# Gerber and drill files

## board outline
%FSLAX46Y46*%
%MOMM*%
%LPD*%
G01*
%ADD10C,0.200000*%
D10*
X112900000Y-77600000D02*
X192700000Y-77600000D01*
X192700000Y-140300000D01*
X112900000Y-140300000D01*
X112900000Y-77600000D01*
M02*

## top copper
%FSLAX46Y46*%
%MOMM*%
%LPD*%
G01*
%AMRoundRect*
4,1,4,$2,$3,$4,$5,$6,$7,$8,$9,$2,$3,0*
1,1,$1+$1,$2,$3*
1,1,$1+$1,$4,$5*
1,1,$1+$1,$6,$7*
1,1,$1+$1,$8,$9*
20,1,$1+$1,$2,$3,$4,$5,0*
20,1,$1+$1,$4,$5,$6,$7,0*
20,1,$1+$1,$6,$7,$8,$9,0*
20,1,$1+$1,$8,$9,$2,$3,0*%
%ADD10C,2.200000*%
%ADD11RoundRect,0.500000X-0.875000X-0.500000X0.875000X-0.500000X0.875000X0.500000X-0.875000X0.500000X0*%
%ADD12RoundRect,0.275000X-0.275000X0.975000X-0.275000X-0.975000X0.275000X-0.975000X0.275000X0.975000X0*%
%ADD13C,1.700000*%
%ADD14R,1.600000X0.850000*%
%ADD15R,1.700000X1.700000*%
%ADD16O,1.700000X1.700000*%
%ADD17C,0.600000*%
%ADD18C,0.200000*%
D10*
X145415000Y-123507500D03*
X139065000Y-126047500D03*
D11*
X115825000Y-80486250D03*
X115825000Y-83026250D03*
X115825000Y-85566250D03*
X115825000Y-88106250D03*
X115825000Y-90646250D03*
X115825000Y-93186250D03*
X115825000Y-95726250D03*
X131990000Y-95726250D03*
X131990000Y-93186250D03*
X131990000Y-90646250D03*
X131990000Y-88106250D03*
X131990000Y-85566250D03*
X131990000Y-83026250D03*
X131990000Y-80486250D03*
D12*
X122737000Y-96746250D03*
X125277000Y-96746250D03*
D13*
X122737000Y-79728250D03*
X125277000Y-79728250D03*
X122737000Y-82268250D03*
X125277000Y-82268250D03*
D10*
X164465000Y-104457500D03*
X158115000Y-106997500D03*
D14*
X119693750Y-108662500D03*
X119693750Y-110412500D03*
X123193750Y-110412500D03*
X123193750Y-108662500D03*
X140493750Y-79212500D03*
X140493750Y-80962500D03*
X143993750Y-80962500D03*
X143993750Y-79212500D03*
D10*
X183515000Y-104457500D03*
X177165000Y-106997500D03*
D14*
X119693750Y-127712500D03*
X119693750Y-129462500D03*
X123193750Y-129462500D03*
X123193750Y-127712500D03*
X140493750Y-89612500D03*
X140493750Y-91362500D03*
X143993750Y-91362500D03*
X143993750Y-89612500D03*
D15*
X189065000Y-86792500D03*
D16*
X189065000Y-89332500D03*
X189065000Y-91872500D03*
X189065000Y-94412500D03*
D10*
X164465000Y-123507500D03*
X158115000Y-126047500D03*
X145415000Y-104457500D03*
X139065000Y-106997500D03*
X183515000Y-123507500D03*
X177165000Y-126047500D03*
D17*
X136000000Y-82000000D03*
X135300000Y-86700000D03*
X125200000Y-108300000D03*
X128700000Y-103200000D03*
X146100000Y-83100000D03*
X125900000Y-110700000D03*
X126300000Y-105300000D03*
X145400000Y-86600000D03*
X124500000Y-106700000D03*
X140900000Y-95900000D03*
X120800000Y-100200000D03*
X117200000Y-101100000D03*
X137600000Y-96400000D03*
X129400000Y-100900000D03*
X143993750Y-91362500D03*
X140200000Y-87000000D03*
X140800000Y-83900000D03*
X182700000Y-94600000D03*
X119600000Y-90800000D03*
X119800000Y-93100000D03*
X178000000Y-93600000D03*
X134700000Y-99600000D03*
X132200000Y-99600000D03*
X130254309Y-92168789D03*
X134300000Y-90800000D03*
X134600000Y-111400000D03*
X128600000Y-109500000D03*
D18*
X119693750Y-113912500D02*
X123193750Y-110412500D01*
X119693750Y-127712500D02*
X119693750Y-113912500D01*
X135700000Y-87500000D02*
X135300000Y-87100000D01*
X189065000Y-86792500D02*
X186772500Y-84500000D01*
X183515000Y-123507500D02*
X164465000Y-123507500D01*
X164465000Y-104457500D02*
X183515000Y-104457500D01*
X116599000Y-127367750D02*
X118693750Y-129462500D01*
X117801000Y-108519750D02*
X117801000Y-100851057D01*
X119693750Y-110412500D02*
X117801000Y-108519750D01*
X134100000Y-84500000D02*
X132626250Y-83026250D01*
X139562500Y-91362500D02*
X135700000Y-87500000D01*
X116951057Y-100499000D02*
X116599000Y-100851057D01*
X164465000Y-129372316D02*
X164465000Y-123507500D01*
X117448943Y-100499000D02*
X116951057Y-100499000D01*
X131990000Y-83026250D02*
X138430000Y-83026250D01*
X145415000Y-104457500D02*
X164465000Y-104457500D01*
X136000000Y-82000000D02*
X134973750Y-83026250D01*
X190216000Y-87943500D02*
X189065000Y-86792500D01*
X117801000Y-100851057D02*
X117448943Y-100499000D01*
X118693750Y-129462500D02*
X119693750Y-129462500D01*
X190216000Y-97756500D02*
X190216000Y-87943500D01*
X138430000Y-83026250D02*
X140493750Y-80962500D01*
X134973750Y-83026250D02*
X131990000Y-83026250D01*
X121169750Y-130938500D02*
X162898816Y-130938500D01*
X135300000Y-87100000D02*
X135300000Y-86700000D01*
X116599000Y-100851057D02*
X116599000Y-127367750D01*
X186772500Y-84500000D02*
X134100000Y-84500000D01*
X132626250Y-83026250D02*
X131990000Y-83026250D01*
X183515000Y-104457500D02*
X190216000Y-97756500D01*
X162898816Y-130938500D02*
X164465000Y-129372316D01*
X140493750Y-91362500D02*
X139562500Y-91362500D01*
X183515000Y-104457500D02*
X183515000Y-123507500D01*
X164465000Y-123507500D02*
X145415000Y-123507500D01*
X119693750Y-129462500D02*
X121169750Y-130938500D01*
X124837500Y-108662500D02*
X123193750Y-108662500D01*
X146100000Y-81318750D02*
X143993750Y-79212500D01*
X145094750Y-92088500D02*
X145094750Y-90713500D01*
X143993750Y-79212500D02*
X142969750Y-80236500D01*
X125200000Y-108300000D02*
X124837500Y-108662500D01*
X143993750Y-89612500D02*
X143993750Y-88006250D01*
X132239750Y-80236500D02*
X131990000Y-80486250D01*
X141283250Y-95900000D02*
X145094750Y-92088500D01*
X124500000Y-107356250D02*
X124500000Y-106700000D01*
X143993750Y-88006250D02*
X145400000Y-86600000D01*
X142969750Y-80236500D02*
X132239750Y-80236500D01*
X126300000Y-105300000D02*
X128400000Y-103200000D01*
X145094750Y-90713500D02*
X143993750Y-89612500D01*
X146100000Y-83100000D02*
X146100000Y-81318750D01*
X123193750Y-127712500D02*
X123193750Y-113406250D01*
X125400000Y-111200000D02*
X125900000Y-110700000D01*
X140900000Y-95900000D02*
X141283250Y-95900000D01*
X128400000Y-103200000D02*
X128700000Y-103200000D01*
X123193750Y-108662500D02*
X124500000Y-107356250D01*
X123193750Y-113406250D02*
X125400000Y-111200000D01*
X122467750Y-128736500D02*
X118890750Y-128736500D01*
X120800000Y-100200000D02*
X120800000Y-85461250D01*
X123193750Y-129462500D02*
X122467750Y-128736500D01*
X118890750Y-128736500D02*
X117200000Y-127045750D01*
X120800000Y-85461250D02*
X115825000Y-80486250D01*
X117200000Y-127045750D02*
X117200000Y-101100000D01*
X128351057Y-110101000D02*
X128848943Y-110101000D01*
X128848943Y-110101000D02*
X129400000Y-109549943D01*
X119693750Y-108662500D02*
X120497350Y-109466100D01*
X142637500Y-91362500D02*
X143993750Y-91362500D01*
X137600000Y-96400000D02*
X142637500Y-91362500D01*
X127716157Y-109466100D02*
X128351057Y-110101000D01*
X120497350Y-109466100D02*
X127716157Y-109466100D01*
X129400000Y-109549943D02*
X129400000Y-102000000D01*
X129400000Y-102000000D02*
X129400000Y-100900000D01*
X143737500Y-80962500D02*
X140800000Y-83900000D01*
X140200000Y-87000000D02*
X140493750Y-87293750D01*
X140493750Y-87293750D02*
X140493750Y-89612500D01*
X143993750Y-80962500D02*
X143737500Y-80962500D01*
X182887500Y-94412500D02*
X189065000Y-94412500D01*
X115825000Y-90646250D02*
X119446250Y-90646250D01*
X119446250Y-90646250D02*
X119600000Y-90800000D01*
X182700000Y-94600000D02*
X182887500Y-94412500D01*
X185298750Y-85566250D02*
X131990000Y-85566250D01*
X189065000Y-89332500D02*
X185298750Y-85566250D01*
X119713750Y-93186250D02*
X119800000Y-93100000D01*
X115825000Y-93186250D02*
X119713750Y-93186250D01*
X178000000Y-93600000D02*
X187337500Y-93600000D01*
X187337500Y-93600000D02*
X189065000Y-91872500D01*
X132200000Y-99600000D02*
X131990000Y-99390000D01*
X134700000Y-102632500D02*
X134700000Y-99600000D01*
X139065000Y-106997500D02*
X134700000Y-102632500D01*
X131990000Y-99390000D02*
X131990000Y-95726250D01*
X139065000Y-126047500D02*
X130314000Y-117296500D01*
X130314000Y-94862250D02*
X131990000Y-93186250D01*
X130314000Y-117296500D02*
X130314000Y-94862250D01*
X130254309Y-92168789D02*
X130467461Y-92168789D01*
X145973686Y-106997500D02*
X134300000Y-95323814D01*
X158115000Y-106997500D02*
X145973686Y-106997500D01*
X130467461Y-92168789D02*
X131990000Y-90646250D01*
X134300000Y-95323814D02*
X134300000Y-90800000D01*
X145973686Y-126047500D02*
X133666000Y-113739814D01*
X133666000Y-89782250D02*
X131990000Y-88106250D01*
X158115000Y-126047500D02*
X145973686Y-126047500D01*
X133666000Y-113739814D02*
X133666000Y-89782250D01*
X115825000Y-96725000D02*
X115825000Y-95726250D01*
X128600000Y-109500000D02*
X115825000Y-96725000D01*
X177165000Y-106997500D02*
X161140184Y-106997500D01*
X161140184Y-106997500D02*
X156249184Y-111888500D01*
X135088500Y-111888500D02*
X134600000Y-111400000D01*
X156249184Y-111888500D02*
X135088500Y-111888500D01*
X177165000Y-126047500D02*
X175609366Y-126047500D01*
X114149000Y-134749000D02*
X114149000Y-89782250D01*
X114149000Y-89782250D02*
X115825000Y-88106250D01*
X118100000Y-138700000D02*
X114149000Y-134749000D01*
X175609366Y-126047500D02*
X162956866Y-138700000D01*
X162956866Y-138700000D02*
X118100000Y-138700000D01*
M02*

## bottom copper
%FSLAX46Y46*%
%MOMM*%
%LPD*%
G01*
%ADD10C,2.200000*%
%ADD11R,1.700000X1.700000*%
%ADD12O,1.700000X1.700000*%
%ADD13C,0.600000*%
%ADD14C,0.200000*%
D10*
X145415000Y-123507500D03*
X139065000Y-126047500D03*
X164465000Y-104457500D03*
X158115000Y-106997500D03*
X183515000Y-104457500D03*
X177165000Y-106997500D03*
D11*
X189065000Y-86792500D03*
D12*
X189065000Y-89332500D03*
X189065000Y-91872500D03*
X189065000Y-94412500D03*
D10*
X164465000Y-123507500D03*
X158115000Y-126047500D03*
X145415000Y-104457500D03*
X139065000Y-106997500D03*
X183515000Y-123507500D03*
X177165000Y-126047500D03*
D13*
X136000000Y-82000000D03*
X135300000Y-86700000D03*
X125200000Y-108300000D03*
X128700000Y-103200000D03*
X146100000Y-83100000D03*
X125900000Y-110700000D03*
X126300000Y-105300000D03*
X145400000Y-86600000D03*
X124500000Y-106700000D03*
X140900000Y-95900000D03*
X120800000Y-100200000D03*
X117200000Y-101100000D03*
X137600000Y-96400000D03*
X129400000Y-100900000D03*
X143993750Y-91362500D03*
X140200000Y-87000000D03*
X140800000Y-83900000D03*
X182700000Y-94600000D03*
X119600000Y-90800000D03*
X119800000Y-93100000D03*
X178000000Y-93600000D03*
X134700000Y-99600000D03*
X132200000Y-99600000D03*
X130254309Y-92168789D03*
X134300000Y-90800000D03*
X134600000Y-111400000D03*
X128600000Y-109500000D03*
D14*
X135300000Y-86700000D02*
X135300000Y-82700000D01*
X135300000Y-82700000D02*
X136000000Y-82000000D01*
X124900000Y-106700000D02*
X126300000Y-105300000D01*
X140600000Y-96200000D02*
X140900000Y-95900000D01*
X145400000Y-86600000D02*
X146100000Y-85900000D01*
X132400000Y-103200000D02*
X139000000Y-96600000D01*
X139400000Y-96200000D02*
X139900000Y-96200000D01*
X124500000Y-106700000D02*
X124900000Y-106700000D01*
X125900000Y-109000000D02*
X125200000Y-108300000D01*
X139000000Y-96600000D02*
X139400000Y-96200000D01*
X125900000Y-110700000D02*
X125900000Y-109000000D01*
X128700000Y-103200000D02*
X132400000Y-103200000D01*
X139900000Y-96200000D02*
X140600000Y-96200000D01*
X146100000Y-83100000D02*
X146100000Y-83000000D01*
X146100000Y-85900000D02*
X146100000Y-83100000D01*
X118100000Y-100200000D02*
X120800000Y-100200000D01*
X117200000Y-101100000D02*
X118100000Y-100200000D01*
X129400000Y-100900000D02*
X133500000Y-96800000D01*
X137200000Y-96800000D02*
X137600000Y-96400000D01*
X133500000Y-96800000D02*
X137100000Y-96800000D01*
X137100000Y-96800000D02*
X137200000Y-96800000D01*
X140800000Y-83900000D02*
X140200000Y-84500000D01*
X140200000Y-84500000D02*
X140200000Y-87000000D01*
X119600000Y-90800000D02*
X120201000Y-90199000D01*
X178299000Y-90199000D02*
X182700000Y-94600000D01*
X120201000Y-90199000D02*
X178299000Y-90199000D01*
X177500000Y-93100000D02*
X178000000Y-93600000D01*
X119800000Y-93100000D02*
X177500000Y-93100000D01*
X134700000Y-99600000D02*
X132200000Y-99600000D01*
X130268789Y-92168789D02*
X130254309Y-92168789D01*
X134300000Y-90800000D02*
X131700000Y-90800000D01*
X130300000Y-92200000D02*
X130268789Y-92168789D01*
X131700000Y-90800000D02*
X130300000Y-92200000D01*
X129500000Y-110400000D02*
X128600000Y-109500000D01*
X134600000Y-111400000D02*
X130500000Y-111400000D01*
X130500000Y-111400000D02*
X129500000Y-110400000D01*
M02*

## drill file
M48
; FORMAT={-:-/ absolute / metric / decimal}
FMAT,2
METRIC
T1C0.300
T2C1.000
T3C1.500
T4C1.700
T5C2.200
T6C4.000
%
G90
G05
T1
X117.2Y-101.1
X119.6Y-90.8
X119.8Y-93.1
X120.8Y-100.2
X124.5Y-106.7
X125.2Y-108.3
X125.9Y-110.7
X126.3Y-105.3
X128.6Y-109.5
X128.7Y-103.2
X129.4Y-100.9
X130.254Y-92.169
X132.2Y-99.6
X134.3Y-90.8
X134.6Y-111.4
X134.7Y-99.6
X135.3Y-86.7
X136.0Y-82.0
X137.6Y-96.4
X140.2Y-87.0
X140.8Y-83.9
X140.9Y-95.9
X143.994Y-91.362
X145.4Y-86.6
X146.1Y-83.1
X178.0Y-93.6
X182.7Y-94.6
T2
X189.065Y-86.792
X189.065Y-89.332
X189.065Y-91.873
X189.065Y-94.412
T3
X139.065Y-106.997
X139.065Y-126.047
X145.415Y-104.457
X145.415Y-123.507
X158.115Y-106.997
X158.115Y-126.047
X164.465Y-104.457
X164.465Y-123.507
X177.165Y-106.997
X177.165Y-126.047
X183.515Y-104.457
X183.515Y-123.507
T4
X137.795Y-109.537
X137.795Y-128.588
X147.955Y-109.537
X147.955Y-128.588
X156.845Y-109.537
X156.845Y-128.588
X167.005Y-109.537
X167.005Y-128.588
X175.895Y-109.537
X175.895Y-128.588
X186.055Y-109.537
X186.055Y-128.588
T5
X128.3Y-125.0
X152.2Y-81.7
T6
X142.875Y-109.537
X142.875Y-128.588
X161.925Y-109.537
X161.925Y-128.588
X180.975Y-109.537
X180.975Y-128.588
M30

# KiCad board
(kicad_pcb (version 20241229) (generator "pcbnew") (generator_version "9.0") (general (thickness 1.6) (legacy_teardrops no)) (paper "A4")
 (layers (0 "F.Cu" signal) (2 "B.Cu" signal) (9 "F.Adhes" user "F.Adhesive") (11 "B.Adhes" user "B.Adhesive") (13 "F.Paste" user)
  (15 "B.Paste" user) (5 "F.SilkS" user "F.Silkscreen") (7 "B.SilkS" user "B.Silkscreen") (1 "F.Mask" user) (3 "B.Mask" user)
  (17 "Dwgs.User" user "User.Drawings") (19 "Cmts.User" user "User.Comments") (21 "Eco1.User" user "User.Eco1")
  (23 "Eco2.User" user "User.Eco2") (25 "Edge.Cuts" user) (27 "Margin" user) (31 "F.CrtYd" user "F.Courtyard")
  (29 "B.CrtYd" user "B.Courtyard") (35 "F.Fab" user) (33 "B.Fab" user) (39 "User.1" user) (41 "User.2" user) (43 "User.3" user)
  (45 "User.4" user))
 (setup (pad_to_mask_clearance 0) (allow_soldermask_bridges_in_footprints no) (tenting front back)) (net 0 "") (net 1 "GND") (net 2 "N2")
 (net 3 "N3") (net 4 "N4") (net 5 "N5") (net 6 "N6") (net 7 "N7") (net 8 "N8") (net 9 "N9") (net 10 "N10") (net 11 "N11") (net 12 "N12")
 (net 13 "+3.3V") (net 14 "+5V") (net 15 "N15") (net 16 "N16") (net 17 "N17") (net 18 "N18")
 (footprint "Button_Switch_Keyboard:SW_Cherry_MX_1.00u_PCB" (layer "F.Cu") (at 145.415 123.5075)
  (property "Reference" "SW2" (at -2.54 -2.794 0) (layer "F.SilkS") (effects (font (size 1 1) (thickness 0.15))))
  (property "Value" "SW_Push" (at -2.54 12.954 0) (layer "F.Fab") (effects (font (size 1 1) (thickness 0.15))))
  (pad "" np_thru_hole circle (at -7.62 5.08) (size 1.7 1.7) (drill 1.7) (layers "*.Cu" "*.Mask"))
  (pad "" np_thru_hole circle (at -2.54 5.08) (size 4 4) (drill 4) (layers "*.Cu" "*.Mask"))
  (pad "" np_thru_hole circle (at 2.54 5.08) (size 1.7 1.7) (drill 1.7) (layers "*.Cu" "*.Mask"))
  (pad "1" thru_hole circle (at 0 0) (size 2.2 2.2) (drill 1.5) (layers "*.Cu" "*.Mask") (remove_unused_layers no) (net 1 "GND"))
  (pad "2" thru_hole circle (at -6.35 2.54) (size 2.2 2.2) (drill 1.5) (layers "*.Cu" "*.Mask") (remove_unused_layers no) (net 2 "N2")))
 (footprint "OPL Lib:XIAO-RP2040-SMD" (layer "F.Cu") (at 123.825 88.10625)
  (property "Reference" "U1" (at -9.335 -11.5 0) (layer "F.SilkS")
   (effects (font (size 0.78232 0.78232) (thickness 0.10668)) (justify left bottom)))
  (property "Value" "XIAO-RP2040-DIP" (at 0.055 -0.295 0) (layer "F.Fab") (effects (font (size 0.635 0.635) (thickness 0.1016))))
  (pad "1" smd roundrect (at -8 -7.62) (size 2.75 2) (layers "F.Cu" "F.Mask" "F.Paste") (roundrect_rratio 0.25) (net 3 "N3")
   (solder_mask_margin 0.0508) (thermal_bridge_angle 45))
  (pad "2" smd roundrect (at -8 -5.08) (size 2.75 2) (layers "F.Cu" "F.Mask" "F.Paste") (roundrect_rratio 0.25) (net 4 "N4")
   (solder_mask_margin 0.0508) (thermal_bridge_angle 45))
  (pad "3" smd roundrect (at -8 -2.54) (size 2.75 2) (layers "F.Cu" "F.Mask" "F.Paste") (roundrect_rratio 0.25) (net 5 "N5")
   (solder_mask_margin 0.0508) (thermal_bridge_angle 45))
  (pad "4" smd roundrect (at -8 0) (size 2.75 2) (layers "F.Cu" "F.Mask" "F.Paste") (roundrect_rratio 0.25) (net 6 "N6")
   (solder_mask_margin 0.0508) (thermal_bridge_angle 45))
  (pad "5" smd roundrect (at -8 2.54) (size 2.75 2) (layers "F.Cu" "F.Mask" "F.Paste") (roundrect_rratio 0.25) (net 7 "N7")
   (solder_mask_margin 0.0508) (thermal_bridge_angle 45))
  (pad "6" smd roundrect (at -8 5.08) (size 2.75 2) (layers "F.Cu" "F.Mask" "F.Paste") (roundrect_rratio 0.25) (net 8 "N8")
   (solder_mask_margin 0.0508) (thermal_bridge_angle 45))
  (pad "7" smd roundrect (at -8 7.62) (size 2.75 2) (layers "F.Cu" "F.Mask" "F.Paste") (roundrect_rratio 0.25) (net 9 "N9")
   (solder_mask_margin 0.0508) (thermal_bridge_angle 45))
  (pad "8" smd roundrect (at 8.165 7.62) (size 2.75 2) (layers "F.Cu" "F.Mask" "F.Paste") (roundrect_rratio 0.25) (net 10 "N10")
   (solder_mask_margin 0.0508) (thermal_bridge_angle 45))
  (pad "9" smd roundrect (at 8.165 5.08) (size 2.75 2) (layers "F.Cu" "F.Mask" "F.Paste") (roundrect_rratio 0.25) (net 2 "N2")
   (solder_mask_margin 0.0508) (thermal_bridge_angle 45))
  (pad "10" smd roundrect (at 8.165 2.54) (size 2.75 2) (layers "F.Cu" "F.Mask" "F.Paste") (roundrect_rratio 0.25) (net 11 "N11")
   (solder_mask_margin 0.0508) (thermal_bridge_angle 45))
  (pad "11" smd roundrect (at 8.165 0) (size 2.75 2) (layers "F.Cu" "F.Mask" "F.Paste") (roundrect_rratio 0.25) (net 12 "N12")
   (solder_mask_margin 0.0508) (thermal_bridge_angle 45))
  (pad "12" smd roundrect (at 8.165 -2.54) (size 2.75 2) (layers "F.Cu" "F.Mask" "F.Paste") (roundrect_rratio 0.25) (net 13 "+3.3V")
   (solder_mask_margin 0.0508) (thermal_bridge_angle 45))
  (pad "13" smd roundrect (at 8.165 -5.08) (size 2.75 2) (layers "F.Cu" "F.Mask" "F.Paste") (roundrect_rratio 0.25) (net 1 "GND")
   (solder_mask_margin 0.0508) (thermal_bridge_angle 45))
  (pad "14" smd roundrect (at 8.165 -7.62) (size 2.75 2) (layers "F.Cu" "F.Mask" "F.Paste") (roundrect_rratio 0.25) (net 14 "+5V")
   (solder_mask_margin 0.0508) (thermal_bridge_angle 45))
  (pad "15" smd roundrect (at -1.088 8.64 270) (size 2.5 1.1) (layers "F.Cu" "F.Mask" "F.Paste") (roundrect_rratio 0.25)
   (thermal_bridge_angle 45))
  (pad "16" smd roundrect (at 1.452 8.64 270) (size 2.5 1.1) (layers "F.Cu" "F.Mask" "F.Paste") (roundrect_rratio 0.25)
   (thermal_bridge_angle 45))
  (pad "17" smd circle (at -1.088 -8.378) (size 1.7 1.7) (layers "F.Cu" "F.Mask" "F.Paste"))
  (pad "18" smd circle (at 1.452 -8.378) (size 1.7 1.7) (layers "F.Cu" "F.Mask" "F.Paste"))
  (pad "19" smd circle (at -1.088 -5.838) (size 1.7 1.7) (layers "F.Cu" "F.Mask" "F.Paste"))
  (pad "20" smd circle (at 1.452 -5.838) (size 1.7 1.7) (layers "F.Cu" "F.Mask" "F.Paste")))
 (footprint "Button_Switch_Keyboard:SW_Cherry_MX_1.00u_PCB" (layer "F.Cu") (at 164.465 104.4575)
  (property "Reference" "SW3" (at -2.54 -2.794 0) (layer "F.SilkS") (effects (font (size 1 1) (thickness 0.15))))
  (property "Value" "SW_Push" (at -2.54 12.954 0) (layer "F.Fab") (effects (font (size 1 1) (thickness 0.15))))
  (pad "" np_thru_hole circle (at -7.62 5.08) (size 1.7 1.7) (drill 1.7) (layers "*.Cu" "*.Mask"))
  (pad "" np_thru_hole circle (at -2.54 5.08) (size 4 4) (drill 4) (layers "*.Cu" "*.Mask"))
  (pad "" np_thru_hole circle (at 2.54 5.08) (size 1.7 1.7) (drill 1.7) (layers "*.Cu" "*.Mask"))
  (pad "1" thru_hole circle (at 0 0) (size 2.2 2.2) (drill 1.5) (layers "*.Cu" "*.Mask") (remove_unused_layers no) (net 1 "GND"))
  (pad "2" thru_hole circle (at -6.35 2.54) (size 2.2 2.2) (drill 1.5) (layers "*.Cu" "*.Mask") (remove_unused_layers no) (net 11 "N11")))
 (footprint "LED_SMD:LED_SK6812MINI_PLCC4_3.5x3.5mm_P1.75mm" (layer "F.Cu") (at 121.44375 109.5375)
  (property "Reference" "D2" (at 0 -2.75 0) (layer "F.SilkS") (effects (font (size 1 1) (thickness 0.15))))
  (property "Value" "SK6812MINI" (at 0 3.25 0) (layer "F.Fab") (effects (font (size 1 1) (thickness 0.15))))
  (pad "1" smd rect (at -1.75 -0.875) (size 1.6 0.85) (layers "F.Cu" "F.Mask" "F.Paste") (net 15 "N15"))
  (pad "2" smd rect (at -1.75 0.875) (size 1.6 0.85) (layers "F.Cu" "F.Mask" "F.Paste") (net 1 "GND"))
  (pad "3" smd rect (at 1.75 0.875) (size 1.6 0.85) (layers "F.Cu" "F.Mask" "F.Paste") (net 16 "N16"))
  (pad "4" smd rect (at 1.75 -0.875) (size 1.6 0.85) (layers "F.Cu" "F.Mask" "F.Paste") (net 14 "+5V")))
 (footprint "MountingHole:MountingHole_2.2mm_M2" (layer "F.Cu") (at 128.3 125)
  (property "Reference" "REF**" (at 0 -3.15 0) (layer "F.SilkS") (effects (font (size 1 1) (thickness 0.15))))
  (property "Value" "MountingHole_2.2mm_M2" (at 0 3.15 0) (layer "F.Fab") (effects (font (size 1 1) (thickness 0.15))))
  (pad "" np_thru_hole circle (at 0 0) (size 2.2 2.2) (drill 2.2) (layers "*.Cu" "*.Mask")))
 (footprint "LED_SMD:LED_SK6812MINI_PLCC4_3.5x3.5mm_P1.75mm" (layer "F.Cu") (at 142.24375 80.0875)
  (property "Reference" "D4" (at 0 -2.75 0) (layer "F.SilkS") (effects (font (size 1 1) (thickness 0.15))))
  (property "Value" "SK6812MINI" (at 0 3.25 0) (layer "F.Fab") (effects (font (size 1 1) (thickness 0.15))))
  (pad "1" smd rect (at -1.75 -0.875) (size 1.6 0.85) (layers "F.Cu" "F.Mask" "F.Paste") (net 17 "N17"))
  (pad "2" smd rect (at -1.75 0.875) (size 1.6 0.85) (layers "F.Cu" "F.Mask" "F.Paste") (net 1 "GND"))
  (pad "3" smd rect (at 1.75 0.875) (size 1.6 0.85) (layers "F.Cu" "F.Mask" "F.Paste") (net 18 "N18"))
  (pad "4" smd rect (at 1.75 -0.875) (size 1.6 0.85) (layers "F.Cu" "F.Mask" "F.Paste") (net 14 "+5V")))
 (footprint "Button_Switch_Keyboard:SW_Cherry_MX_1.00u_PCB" (layer "F.Cu") (at 183.515 104.4575)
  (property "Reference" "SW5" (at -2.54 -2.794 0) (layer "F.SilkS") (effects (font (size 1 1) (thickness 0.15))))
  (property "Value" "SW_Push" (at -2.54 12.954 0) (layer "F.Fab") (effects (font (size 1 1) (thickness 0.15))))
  (pad "" np_thru_hole circle (at -7.62 5.08) (size 1.7 1.7) (drill 1.7) (layers "*.Cu" "*.Mask"))
  (pad "" np_thru_hole circle (at -2.54 5.08) (size 4 4) (drill 4) (layers "*.Cu" "*.Mask"))
  (pad "" np_thru_hole circle (at 2.54 5.08) (size 1.7 1.7) (drill 1.7) (layers "*.Cu" "*.Mask"))
  (pad "1" thru_hole circle (at 0 0) (size 2.2 2.2) (drill 1.5) (layers "*.Cu" "*.Mask") (remove_unused_layers no) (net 1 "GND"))
  (pad "2" thru_hole circle (at -6.35 2.54) (size 2.2 2.2) (drill 1.5) (layers "*.Cu" "*.Mask") (remove_unused_layers no) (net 9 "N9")))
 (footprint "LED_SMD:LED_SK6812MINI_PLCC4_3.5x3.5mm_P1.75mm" (layer "F.Cu") (at 121.44375 128.5875)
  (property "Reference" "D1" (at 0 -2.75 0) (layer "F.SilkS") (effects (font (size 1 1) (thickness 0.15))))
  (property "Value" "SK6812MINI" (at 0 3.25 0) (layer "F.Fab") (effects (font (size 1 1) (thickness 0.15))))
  (pad "1" smd rect (at -1.75 -0.875) (size 1.6 0.85) (layers "F.Cu" "F.Mask" "F.Paste") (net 16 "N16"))
  (pad "2" smd rect (at -1.75 0.875) (size 1.6 0.85) (layers "F.Cu" "F.Mask" "F.Paste") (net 1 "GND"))
  (pad "3" smd rect (at 1.75 0.875) (size 1.6 0.85) (layers "F.Cu" "F.Mask" "F.Paste") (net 3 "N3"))
  (pad "4" smd rect (at 1.75 -0.875) (size 1.6 0.85) (layers "F.Cu" "F.Mask" "F.Paste") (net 14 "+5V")))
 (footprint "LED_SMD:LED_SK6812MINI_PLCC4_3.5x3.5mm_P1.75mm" (layer "F.Cu") (at 142.24375 90.4875)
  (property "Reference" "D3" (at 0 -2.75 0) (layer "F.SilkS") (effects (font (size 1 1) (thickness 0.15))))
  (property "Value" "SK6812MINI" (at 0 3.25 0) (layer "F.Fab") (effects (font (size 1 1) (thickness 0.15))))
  (pad "1" smd rect (at -1.75 -0.875) (size 1.6 0.85) (layers "F.Cu" "F.Mask" "F.Paste") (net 18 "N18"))
  (pad "2" smd rect (at -1.75 0.875) (size 1.6 0.85) (layers "F.Cu" "F.Mask" "F.Paste") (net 1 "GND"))
  (pad "3" smd rect (at 1.75 0.875) (size 1.6 0.85) (layers "F.Cu" "F.Mask" "F.Paste") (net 15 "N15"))
  (pad "4" smd rect (at 1.75 -0.875) (size 1.6 0.85) (layers "F.Cu" "F.Mask" "F.Paste") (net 14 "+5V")))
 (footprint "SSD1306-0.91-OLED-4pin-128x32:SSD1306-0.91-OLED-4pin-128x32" (layer "F.Cu") (at 152.565 84.6025)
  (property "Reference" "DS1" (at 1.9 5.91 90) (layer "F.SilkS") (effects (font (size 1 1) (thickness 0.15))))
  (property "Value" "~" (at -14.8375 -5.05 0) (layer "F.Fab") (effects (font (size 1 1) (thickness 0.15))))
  (pad "1" thru_hole rect (at 36.5 2.19) (size 1.7 1.7) (drill 1) (layers "*.Cu" "*.Mask") (remove_unused_layers no) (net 1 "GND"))
  (pad "2" thru_hole oval (at 36.5 4.73) (size 1.7 1.7) (drill 1) (layers "*.Cu" "*.Mask") (remove_unused_layers no) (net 13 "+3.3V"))
  (pad "3" thru_hole oval (at 36.5 7.27) (size 1.7 1.7) (drill 1) (layers "*.Cu" "*.Mask") (remove_unused_layers no) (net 8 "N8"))
  (pad "4" thru_hole oval (at 36.5 9.81) (size 1.7 1.7) (drill 1) (layers "*.Cu" "*.Mask") (remove_unused_layers no) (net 7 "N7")))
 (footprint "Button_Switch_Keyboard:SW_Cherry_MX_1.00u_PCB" (layer "F.Cu") (at 164.465 123.5075)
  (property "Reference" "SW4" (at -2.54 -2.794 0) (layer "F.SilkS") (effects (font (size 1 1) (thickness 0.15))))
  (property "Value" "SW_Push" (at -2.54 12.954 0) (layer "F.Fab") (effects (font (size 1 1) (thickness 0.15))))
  (pad "" np_thru_hole circle (at -7.62 5.08) (size 1.7 1.7) (drill 1.7) (layers "*.Cu" "*.Mask"))
  (pad "" np_thru_hole circle (at -2.54 5.08) (size 4 4) (drill 4) (layers "*.Cu" "*.Mask"))
  (pad "" np_thru_hole circle (at 2.54 5.08) (size 1.7 1.7) (drill 1.7) (layers "*.Cu" "*.Mask"))
  (pad "1" thru_hole circle (at 0 0) (size 2.2 2.2) (drill 1.5) (layers "*.Cu" "*.Mask") (remove_unused_layers no) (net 1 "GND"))
  (pad "2" thru_hole circle (at -6.35 2.54) (size 2.2 2.2) (drill 1.5) (layers "*.Cu" "*.Mask") (remove_unused_layers no) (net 12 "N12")))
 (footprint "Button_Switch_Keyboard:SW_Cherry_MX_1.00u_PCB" (layer "F.Cu") (at 145.415 104.4575)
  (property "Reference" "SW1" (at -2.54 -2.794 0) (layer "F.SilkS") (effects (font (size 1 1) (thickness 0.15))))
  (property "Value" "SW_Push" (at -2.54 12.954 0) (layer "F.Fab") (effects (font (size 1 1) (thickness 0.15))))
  (pad "" np_thru_hole circle (at -7.62 5.08) (size 1.7 1.7) (drill 1.7) (layers "*.Cu" "*.Mask"))
  (pad "" np_thru_hole circle (at -2.54 5.08) (size 4 4) (drill 4) (layers "*.Cu" "*.Mask"))
  (pad "" np_thru_hole circle (at 2.54 5.08) (size 1.7 1.7) (drill 1.7) (layers "*.Cu" "*.Mask"))
  (pad "1" thru_hole circle (at 0 0) (size 2.2 2.2) (drill 1.5) (layers "*.Cu" "*.Mask") (remove_unused_layers no) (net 1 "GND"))
  (pad "2" thru_hole circle (at -6.35 2.54) (size 2.2 2.2) (drill 1.5) (layers "*.Cu" "*.Mask") (remove_unused_layers no) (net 10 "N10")))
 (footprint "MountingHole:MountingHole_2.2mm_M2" (layer "F.Cu") (at 152.2 81.7)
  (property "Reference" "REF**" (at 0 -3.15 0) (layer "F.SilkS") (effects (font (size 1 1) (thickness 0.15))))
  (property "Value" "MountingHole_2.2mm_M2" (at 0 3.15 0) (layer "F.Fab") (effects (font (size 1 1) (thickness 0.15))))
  (pad "" np_thru_hole circle (at 0 0) (size 2.2 2.2) (drill 2.2) (layers "*.Cu" "*.Mask")))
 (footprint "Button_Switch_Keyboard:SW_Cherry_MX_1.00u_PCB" (layer "F.Cu") (at 183.515 123.5075)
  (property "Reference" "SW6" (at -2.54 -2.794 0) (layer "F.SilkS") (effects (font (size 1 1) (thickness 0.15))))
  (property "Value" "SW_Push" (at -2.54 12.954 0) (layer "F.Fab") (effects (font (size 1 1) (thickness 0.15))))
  (pad "" np_thru_hole circle (at -7.62 5.08) (size 1.7 1.7) (drill 1.7) (layers "*.Cu" "*.Mask"))
  (pad "" np_thru_hole circle (at -2.54 5.08) (size 4 4) (drill 4) (layers "*.Cu" "*.Mask"))
  (pad "" np_thru_hole circle (at 2.54 5.08) (size 1.7 1.7) (drill 1.7) (layers "*.Cu" "*.Mask"))
  (pad "1" thru_hole circle (at 0 0) (size 2.2 2.2) (drill 1.5) (layers "*.Cu" "*.Mask") (remove_unused_layers no) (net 1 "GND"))
  (pad "2" thru_hole circle (at -6.35 2.54) (size 2.2 2.2) (drill 1.5) (layers "*.Cu" "*.Mask") (remove_unused_layers no) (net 6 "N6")))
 (gr_rect (start 112.9 77.6) (end 192.7 140.3) (stroke (width 0.2) (type solid)) (fill no) (layer "Edge.Cuts"))
 (segment (start 119.69375 113.9125) (end 123.19375 110.4125) (width 0.2) (layer "F.Cu") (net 16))
 (segment (start 119.69375 127.7125) (end 119.69375 113.9125) (width 0.2) (layer "F.Cu") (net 16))
 (segment (start 135.7 87.5) (end 135.3 87.1) (width 0.2) (layer "F.Cu") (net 1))
 (segment (start 189.065 86.7925) (end 186.7725 84.5) (width 0.2) (layer "F.Cu") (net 1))
 (segment (start 183.515 123.5075) (end 164.465 123.5075) (width 0.2) (layer "F.Cu") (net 1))
 (segment (start 164.465 104.4575) (end 183.515 104.4575) (width 0.2) (layer "F.Cu") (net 1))
 (segment (start 116.599 127.36775) (end 118.69375 129.4625) (width 0.2) (layer "F.Cu") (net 1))
 (segment (start 117.801 108.51975) (end 117.801 100.851057) (width 0.2) (layer "F.Cu") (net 1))
 (segment (start 119.69375 110.4125) (end 117.801 108.51975) (width 0.2) (layer "F.Cu") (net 1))
 (segment (start 134.1 84.5) (end 132.62625 83.02625) (width 0.2) (layer "F.Cu") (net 1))
 (segment (start 139.5625 91.3625) (end 135.7 87.5) (width 0.2) (layer "F.Cu") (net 1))
 (segment (start 116.951057 100.499) (end 116.599 100.851057) (width 0.2) (layer "F.Cu") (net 1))
 (segment (start 164.465 129.372316) (end 164.465 123.5075) (width 0.2) (layer "F.Cu") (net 1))
 (segment (start 117.448943 100.499) (end 116.951057 100.499) (width 0.2) (layer "F.Cu") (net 1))
 (segment (start 131.99 83.02625) (end 138.43 83.02625) (width 0.2) (layer "F.Cu") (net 1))
 (segment (start 145.415 104.4575) (end 164.465 104.4575) (width 0.2) (layer "F.Cu") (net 1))
 (segment (start 136 82) (end 134.97375 83.02625) (width 0.2) (layer "F.Cu") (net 1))
 (segment (start 190.216 87.9435) (end 189.065 86.7925) (width 0.2) (layer "F.Cu") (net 1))
 (segment (start 117.801 100.851057) (end 117.448943 100.499) (width 0.2) (layer "F.Cu") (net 1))
 (segment (start 118.69375 129.4625) (end 119.69375 129.4625) (width 0.2) (layer "F.Cu") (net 1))
 (segment (start 190.216 97.7565) (end 190.216 87.9435) (width 0.2) (layer "F.Cu") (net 1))
 (segment (start 138.43 83.02625) (end 140.49375 80.9625) (width 0.2) (layer "F.Cu") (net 1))
 (segment (start 134.97375 83.02625) (end 131.99 83.02625) (width 0.2) (layer "F.Cu") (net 1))
 (segment (start 121.16975 130.9385) (end 162.898816 130.9385) (width 0.2) (layer "F.Cu") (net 1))
 (segment (start 135.3 87.1) (end 135.3 86.7) (width 0.2) (layer "F.Cu") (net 1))
 (segment (start 116.599 100.851057) (end 116.599 127.36775) (width 0.2) (layer "F.Cu") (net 1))
 (segment (start 186.7725 84.5) (end 134.1 84.5) (width 0.2) (layer "F.Cu") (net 1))
 (segment (start 132.62625 83.02625) (end 131.99 83.02625) (width 0.2) (layer "F.Cu") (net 1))
 (segment (start 183.515 104.4575) (end 190.216 97.7565) (width 0.2) (layer "F.Cu") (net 1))
 (segment (start 162.898816 130.9385) (end 164.465 129.372316) (width 0.2) (layer "F.Cu") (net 1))
 (segment (start 140.49375 91.3625) (end 139.5625 91.3625) (width 0.2) (layer "F.Cu") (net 1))
 (segment (start 183.515 104.4575) (end 183.515 123.5075) (width 0.2) (layer "F.Cu") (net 1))
 (segment (start 164.465 123.5075) (end 145.415 123.5075) (width 0.2) (layer "F.Cu") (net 1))
 (segment (start 119.69375 129.4625) (end 121.16975 130.9385) (width 0.2) (layer "F.Cu") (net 1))
 (via (at 136 82) (size 0.6) (drill 0.3) (layers "F.Cu" "B.Cu") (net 1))
 (via (at 135.3 86.7) (size 0.6) (drill 0.3) (layers "F.Cu" "B.Cu") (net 1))
 (segment (start 135.3 86.7) (end 135.3 82.7) (width 0.2) (layer "B.Cu") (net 1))
 (segment (start 135.3 82.7) (end 136 82) (width 0.2) (layer "B.Cu") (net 1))
 (segment (start 124.8375 108.6625) (end 123.19375 108.6625) (width 0.2) (layer "F.Cu") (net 14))
 (segment (start 146.1 81.31875) (end 143.99375 79.2125) (width 0.2) (layer "F.Cu") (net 14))
 (segment (start 145.09475 92.0885) (end 145.09475 90.7135) (width 0.2) (layer "F.Cu") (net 14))
 (segment (start 143.99375 79.2125) (end 142.96975 80.2365) (width 0.2) (layer "F.Cu") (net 14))
 (segment (start 125.2 108.3) (end 124.8375 108.6625) (width 0.2) (layer "F.Cu") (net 14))
 (segment (start 143.99375 89.6125) (end 143.99375 88.00625) (width 0.2) (layer "F.Cu") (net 14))
 (segment (start 132.23975 80.2365) (end 131.99 80.48625) (width 0.2) (layer "F.Cu") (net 14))
 (segment (start 141.28325 95.9) (end 145.09475 92.0885) (width 0.2) (layer "F.Cu") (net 14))
 (segment (start 124.5 107.35625) (end 124.5 106.7) (width 0.2) (layer "F.Cu") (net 14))
 (segment (start 143.99375 88.00625) (end 145.4 86.6) (width 0.2) (layer "F.Cu") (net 14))
 (segment (start 142.96975 80.2365) (end 132.23975 80.2365) (width 0.2) (layer "F.Cu") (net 14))
 (segment (start 126.3 105.3) (end 128.4 103.2) (width 0.2) (layer "F.Cu") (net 14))
 (segment (start 145.09475 90.7135) (end 143.99375 89.6125) (width 0.2) (layer "F.Cu") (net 14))
 (segment (start 146.1 83.1) (end 146.1 81.31875) (width 0.2) (layer "F.Cu") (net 14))
 (segment (start 123.19375 127.7125) (end 123.19375 113.40625) (width 0.2) (layer "F.Cu") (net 14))
 (segment (start 125.4 111.2) (end 125.9 110.7) (width 0.2) (layer "F.Cu") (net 14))
 (segment (start 140.9 95.9) (end 141.28325 95.9) (width 0.2) (layer "F.Cu") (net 14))
 (segment (start 128.4 103.2) (end 128.7 103.2) (width 0.2) (layer "F.Cu") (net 14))
 (segment (start 123.19375 108.6625) (end 124.5 107.35625) (width 0.2) (layer "F.Cu") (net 14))
 (segment (start 123.19375 113.40625) (end 125.4 111.2) (width 0.2) (layer "F.Cu") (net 14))
 (via (at 125.2 108.3) (size 0.6) (drill 0.3) (layers "F.Cu" "B.Cu") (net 14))
 (via (at 128.7 103.2) (size 0.6) (drill 0.3) (layers "F.Cu" "B.Cu") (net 14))
 (via (at 146.1 83.1) (size 0.6) (drill 0.3) (layers "F.Cu" "B.Cu") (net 14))
 (via (at 125.9 110.7) (size 0.6) (drill 0.3) (layers "F.Cu" "B.Cu") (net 14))
 (via (at 126.3 105.3) (size 0.6) (drill 0.3) (layers "F.Cu" "B.Cu") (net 14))
 (via (at 145.4 86.6) (size 0.6) (drill 0.3) (layers "F.Cu" "B.Cu") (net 14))
 (via (at 124.5 106.7) (size 0.6) (drill 0.3) (layers "F.Cu" "B.Cu") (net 14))
 (via (at 140.9 95.9) (size 0.6) (drill 0.3) (layers "F.Cu" "B.Cu") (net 14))
 (segment (start 124.9 106.7) (end 126.3 105.3) (width 0.2) (layer "B.Cu") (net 14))
 (segment (start 140.6 96.2) (end 140.9 95.9) (width 0.2) (layer "B.Cu") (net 14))
 (segment (start 145.4 86.6) (end 146.1 85.9) (width 0.2) (layer "B.Cu") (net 14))
 (segment (start 132.4 103.2) (end 139 96.6) (width 0.2) (layer "B.Cu") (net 14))
 (segment (start 139.4 96.2) (end 139.9 96.2) (width 0.2) (layer "B.Cu") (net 14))
 (segment (start 124.5 106.7) (end 124.9 106.7) (width 0.2) (layer "B.Cu") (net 14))
 (segment (start 125.9 109) (end 125.2 108.3) (width 0.2) (layer "B.Cu") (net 14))
 (segment (start 139 96.6) (end 139.4 96.2) (width 0.2) (layer "B.Cu") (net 14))
 (segment (start 125.9 110.7) (end 125.9 109) (width 0.2) (layer "B.Cu") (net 14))
 (segment (start 128.7 103.2) (end 132.4 103.2) (width 0.2) (layer "B.Cu") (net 14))
 (segment (start 139.9 96.2) (end 140.6 96.2) (width 0.2) (layer "B.Cu") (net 14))
 (segment (start 146.1 83.1) (end 146.1 83) (width 0.2) (layer "B.Cu") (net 14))
 (segment (start 146.1 85.9) (end 146.1 83.1) (width 0.2) (layer "B.Cu") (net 14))
 (segment (start 122.46775 128.7365) (end 118.89075 128.7365) (width 0.2) (layer "F.Cu") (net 3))
 (segment (start 120.8 100.2) (end 120.8 85.46125) (width 0.2) (layer "F.Cu") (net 3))
 (segment (start 123.19375 129.4625) (end 122.46775 128.7365) (width 0.2) (layer "F.Cu") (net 3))
 (segment (start 118.89075 128.7365) (end 117.2 127.04575) (width 0.2) (layer "F.Cu") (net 3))
 (segment (start 120.8 85.46125) (end 115.825 80.48625) (width 0.2) (layer "F.Cu") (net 3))
 (segment (start 117.2 127.04575) (end 117.2 101.1) (width 0.2) (layer "F.Cu") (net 3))
 (via (at 120.8 100.2) (size 0.6) (drill 0.3) (layers "F.Cu" "B.Cu") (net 3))
 (via (at 117.2 101.1) (size 0.6) (drill 0.3) (layers "F.Cu" "B.Cu") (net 3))
 (segment (start 118.1 100.2) (end 120.8 100.2) (width 0.2) (layer "B.Cu") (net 3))
 (segment (start 117.2 101.1) (end 118.1 100.2) (width 0.2) (layer "B.Cu") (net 3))
 (segment (start 128.351057 110.101) (end 128.848943 110.101) (width 0.2) (layer "F.Cu") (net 15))
 (segment (start 128.848943 110.101) (end 129.4 109.549943) (width 0.2) (layer "F.Cu") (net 15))
 (segment (start 119.69375 108.6625) (end 120.49735 109.4661) (width 0.2) (layer "F.Cu") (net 15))
 (segment (start 142.6375 91.3625) (end 143.99375 91.3625) (width 0.2) (layer "F.Cu") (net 15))
 (segment (start 137.6 96.4) (end 142.6375 91.3625) (width 0.2) (layer "F.Cu") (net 15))
 (segment (start 127.716157 109.4661) (end 128.351057 110.101) (width 0.2) (layer "F.Cu") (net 15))
 (segment (start 120.49735 109.4661) (end 127.716157 109.4661) (width 0.2) (layer "F.Cu") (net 15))
 (segment (start 129.4 109.549943) (end 129.4 102) (width 0.2) (layer "F.Cu") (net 15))
 (segment (start 129.4 102) (end 129.4 100.9) (width 0.2) (layer "F.Cu") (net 15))
 (via (at 137.6 96.4) (size 0.6) (drill 0.3) (layers "F.Cu" "B.Cu") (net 15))
 (via (at 129.4 100.9) (size 0.6) (drill 0.3) (layers "F.Cu" "B.Cu") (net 15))
 (via (at 143.99375 91.3625) (size 0.6) (drill 0.3) (layers "F.Cu" "B.Cu") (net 15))
 (segment (start 129.4 100.9) (end 133.5 96.8) (width 0.2) (layer "B.Cu") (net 15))
 (segment (start 137.2 96.8) (end 137.6 96.4) (width 0.2) (layer "B.Cu") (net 15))
 (segment (start 133.5 96.8) (end 137.1 96.8) (width 0.2) (layer "B.Cu") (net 15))
 (segment (start 137.1 96.8) (end 137.2 96.8) (width 0.2) (layer "B.Cu") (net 15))
 (segment (start 143.7375 80.9625) (end 140.8 83.9) (width 0.2) (layer "F.Cu") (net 18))
 (segment (start 140.2 87) (end 140.49375 87.29375) (width 0.2) (layer "F.Cu") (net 18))
 (segment (start 140.49375 87.29375) (end 140.49375 89.6125) (width 0.2) (layer "F.Cu") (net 18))
 (segment (start 143.99375 80.9625) (end 143.7375 80.9625) (width 0.2) (layer "F.Cu") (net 18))
 (via (at 140.2 87) (size 0.6) (drill 0.3) (layers "F.Cu" "B.Cu") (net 18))
 (via (at 140.8 83.9) (size 0.6) (drill 0.3) (layers "F.Cu" "B.Cu") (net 18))
 (segment (start 140.8 83.9) (end 140.2 84.5) (width 0.2) (layer "B.Cu") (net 18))
 (segment (start 140.2 84.5) (end 140.2 87) (width 0.2) (layer "B.Cu") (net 18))
 (segment (start 182.8875 94.4125) (end 189.065 94.4125) (width 0.2) (layer "F.Cu") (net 7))
 (segment (start 115.825 90.64625) (end 119.44625 90.64625) (width 0.2) (layer "F.Cu") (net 7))
 (segment (start 119.44625 90.64625) (end 119.6 90.8) (width 0.2) (layer "F.Cu") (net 7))
 (segment (start 182.7 94.6) (end 182.8875 94.4125) (width 0.2) (layer "F.Cu") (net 7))
 (via (at 182.7 94.6) (size 0.6) (drill 0.3) (layers "F.Cu" "B.Cu") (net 7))
 (via (at 119.6 90.8) (size 0.6) (drill 0.3) (layers "F.Cu" "B.Cu") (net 7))
 (segment (start 119.6 90.8) (end 120.201 90.199) (width 0.2) (layer "B.Cu") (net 7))
 (segment (start 178.299 90.199) (end 182.7 94.6) (width 0.2) (layer "B.Cu") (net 7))
 (segment (start 120.201 90.199) (end 178.299 90.199) (width 0.2) (layer "B.Cu") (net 7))
 (segment (start 185.29875 85.56625) (end 131.99 85.56625) (width 0.2) (layer "F.Cu") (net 13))
 (segment (start 189.065 89.3325) (end 185.29875 85.56625) (width 0.2) (layer "F.Cu") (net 13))
 (segment (start 119.71375 93.18625) (end 119.8 93.1) (width 0.2) (layer "F.Cu") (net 8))
 (segment (start 115.825 93.18625) (end 119.71375 93.18625) (width 0.2) (layer "F.Cu") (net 8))
 (segment (start 178 93.6) (end 187.3375 93.6) (width 0.2) (layer "F.Cu") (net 8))
 (segment (start 187.3375 93.6) (end 189.065 91.8725) (width 0.2) (layer "F.Cu") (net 8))
 (via (at 119.8 93.1) (size 0.6) (drill 0.3) (layers "F.Cu" "B.Cu") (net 8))
 (via (at 178 93.6) (size 0.6) (drill 0.3) (layers "F.Cu" "B.Cu") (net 8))
 (segment (start 177.5 93.1) (end 178 93.6) (width 0.2) (layer "B.Cu") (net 8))
 (segment (start 119.8 93.1) (end 177.5 93.1) (width 0.2) (layer "B.Cu") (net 8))
 (segment (start 132.2 99.6) (end 131.99 99.39) (width 0.2) (layer "F.Cu") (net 10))
 (segment (start 134.7 102.6325) (end 134.7 99.6) (width 0.2) (layer "F.Cu") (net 10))
 (segment (start 139.065 106.9975) (end 134.7 102.6325) (width 0.2) (layer "F.Cu") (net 10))
 (segment (start 131.99 99.39) (end 131.99 95.72625) (width 0.2) (layer "F.Cu") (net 10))
 (via (at 134.7 99.6) (size 0.6) (drill 0.3) (layers "F.Cu" "B.Cu") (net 10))
 (via (at 132.2 99.6) (size 0.6) (drill 0.3) (layers "F.Cu" "B.Cu") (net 10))
 (segment (start 134.7 99.6) (end 132.2 99.6) (width 0.2) (layer "B.Cu") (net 10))
 (segment (start 139.065 126.0475) (end 130.314 117.2965) (width 0.2) (layer "F.Cu") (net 2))
 (segment (start 130.314 94.86225) (end 131.99 93.18625) (width 0.2) (layer "F.Cu") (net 2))
 (segment (start 130.314 117.2965) (end 130.314 94.86225) (width 0.2) (layer "F.Cu") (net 2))
 (segment (start 130.254309 92.168789) (end 130.467461 92.168789) (width 0.2) (layer "F.Cu") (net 11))
 (segment (start 145.973686 106.9975) (end 134.3 95.323814) (width 0.2) (layer "F.Cu") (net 11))
 (segment (start 158.115 106.9975) (end 145.973686 106.9975) (width 0.2) (layer "F.Cu") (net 11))
 (segment (start 130.467461 92.168789) (end 131.99 90.64625) (width 0.2) (layer "F.Cu") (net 11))
 (segment (start 134.3 95.323814) (end 134.3 90.8) (width 0.2) (layer "F.Cu") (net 11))
 (via (at 130.254309 92.168789) (size 0.6) (drill 0.3) (layers "F.Cu" "B.Cu") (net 11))
 (via (at 134.3 90.8) (size 0.6) (drill 0.3) (layers "F.Cu" "B.Cu") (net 11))
 (segment (start 130.268789 92.168789) (end 130.254309 92.168789) (width 0.2) (layer "B.Cu") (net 11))
 (segment (start 134.3 90.8) (end 131.7 90.8) (width 0.2) (layer "B.Cu") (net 11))
 (segment (start 130.3 92.2) (end 130.268789 92.168789) (width 0.2) (layer "B.Cu") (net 11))
 (segment (start 131.7 90.8) (end 130.3 92.2) (width 0.2) (layer "B.Cu") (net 11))
 (segment (start 145.973686 126.0475) (end 133.666 113.739814) (width 0.2) (layer "F.Cu") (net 12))
 (segment (start 133.666 89.78225) (end 131.99 88.10625) (width 0.2) (layer "F.Cu") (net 12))
 (segment (start 158.115 126.0475) (end 145.973686 126.0475) (width 0.2) (layer "F.Cu") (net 12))
 (segment (start 133.666 113.739814) (end 133.666 89.78225) (width 0.2) (layer "F.Cu") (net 12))
 (segment (start 115.825 96.725) (end 115.825 95.72625) (width 0.2) (layer "F.Cu") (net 9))
 (segment (start 128.6 109.5) (end 115.825 96.725) (width 0.2) (layer "F.Cu") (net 9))
 (segment (start 177.165 106.9975) (end 161.140184 106.9975) (width 0.2) (layer "F.Cu") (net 9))
 (segment (start 161.140184 106.9975) (end 156.249184 111.8885) (width 0.2) (layer "F.Cu") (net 9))
 (segment (start 135.0885 111.8885) (end 134.6 111.4) (width 0.2) (layer "F.Cu") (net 9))
 (segment (start 156.249184 111.8885) (end 135.0885 111.8885) (width 0.2) (layer "F.Cu") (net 9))
 (via (at 134.6 111.4) (size 0.6) (drill 0.3) (layers "F.Cu" "B.Cu") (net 9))
 (via (at 128.6 109.5) (size 0.6) (drill 0.3) (layers "F.Cu" "B.Cu") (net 9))
 (segment (start 129.5 110.4) (end 128.6 109.5) (width 0.2) (layer "B.Cu") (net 9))
 (segment (start 134.6 111.4) (end 130.5 111.4) (width 0.2) (layer "B.Cu") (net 9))
 (segment (start 130.5 111.4) (end 129.5 110.4) (width 0.2) (layer "B.Cu") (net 9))
 (segment (start 177.165 126.0475) (end 175.609366 126.0475) (width 0.2) (layer "F.Cu") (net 6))
 (segment (start 114.149 134.749) (end 114.149 89.78225) (width 0.2) (layer "F.Cu") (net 6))
 (segment (start 114.149 89.78225) (end 115.825 88.10625) (width 0.2) (layer "F.Cu") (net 6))
 (segment (start 118.1 138.7) (end 114.149 134.749) (width 0.2) (layer "F.Cu") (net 6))
 (segment (start 175.609366 126.0475) (end 162.956866 138.7) (width 0.2) (layer "F.Cu") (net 6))
 (segment (start 162.956866 138.7) (end 118.1 138.7) (width 0.2) (layer "F.Cu") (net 6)))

